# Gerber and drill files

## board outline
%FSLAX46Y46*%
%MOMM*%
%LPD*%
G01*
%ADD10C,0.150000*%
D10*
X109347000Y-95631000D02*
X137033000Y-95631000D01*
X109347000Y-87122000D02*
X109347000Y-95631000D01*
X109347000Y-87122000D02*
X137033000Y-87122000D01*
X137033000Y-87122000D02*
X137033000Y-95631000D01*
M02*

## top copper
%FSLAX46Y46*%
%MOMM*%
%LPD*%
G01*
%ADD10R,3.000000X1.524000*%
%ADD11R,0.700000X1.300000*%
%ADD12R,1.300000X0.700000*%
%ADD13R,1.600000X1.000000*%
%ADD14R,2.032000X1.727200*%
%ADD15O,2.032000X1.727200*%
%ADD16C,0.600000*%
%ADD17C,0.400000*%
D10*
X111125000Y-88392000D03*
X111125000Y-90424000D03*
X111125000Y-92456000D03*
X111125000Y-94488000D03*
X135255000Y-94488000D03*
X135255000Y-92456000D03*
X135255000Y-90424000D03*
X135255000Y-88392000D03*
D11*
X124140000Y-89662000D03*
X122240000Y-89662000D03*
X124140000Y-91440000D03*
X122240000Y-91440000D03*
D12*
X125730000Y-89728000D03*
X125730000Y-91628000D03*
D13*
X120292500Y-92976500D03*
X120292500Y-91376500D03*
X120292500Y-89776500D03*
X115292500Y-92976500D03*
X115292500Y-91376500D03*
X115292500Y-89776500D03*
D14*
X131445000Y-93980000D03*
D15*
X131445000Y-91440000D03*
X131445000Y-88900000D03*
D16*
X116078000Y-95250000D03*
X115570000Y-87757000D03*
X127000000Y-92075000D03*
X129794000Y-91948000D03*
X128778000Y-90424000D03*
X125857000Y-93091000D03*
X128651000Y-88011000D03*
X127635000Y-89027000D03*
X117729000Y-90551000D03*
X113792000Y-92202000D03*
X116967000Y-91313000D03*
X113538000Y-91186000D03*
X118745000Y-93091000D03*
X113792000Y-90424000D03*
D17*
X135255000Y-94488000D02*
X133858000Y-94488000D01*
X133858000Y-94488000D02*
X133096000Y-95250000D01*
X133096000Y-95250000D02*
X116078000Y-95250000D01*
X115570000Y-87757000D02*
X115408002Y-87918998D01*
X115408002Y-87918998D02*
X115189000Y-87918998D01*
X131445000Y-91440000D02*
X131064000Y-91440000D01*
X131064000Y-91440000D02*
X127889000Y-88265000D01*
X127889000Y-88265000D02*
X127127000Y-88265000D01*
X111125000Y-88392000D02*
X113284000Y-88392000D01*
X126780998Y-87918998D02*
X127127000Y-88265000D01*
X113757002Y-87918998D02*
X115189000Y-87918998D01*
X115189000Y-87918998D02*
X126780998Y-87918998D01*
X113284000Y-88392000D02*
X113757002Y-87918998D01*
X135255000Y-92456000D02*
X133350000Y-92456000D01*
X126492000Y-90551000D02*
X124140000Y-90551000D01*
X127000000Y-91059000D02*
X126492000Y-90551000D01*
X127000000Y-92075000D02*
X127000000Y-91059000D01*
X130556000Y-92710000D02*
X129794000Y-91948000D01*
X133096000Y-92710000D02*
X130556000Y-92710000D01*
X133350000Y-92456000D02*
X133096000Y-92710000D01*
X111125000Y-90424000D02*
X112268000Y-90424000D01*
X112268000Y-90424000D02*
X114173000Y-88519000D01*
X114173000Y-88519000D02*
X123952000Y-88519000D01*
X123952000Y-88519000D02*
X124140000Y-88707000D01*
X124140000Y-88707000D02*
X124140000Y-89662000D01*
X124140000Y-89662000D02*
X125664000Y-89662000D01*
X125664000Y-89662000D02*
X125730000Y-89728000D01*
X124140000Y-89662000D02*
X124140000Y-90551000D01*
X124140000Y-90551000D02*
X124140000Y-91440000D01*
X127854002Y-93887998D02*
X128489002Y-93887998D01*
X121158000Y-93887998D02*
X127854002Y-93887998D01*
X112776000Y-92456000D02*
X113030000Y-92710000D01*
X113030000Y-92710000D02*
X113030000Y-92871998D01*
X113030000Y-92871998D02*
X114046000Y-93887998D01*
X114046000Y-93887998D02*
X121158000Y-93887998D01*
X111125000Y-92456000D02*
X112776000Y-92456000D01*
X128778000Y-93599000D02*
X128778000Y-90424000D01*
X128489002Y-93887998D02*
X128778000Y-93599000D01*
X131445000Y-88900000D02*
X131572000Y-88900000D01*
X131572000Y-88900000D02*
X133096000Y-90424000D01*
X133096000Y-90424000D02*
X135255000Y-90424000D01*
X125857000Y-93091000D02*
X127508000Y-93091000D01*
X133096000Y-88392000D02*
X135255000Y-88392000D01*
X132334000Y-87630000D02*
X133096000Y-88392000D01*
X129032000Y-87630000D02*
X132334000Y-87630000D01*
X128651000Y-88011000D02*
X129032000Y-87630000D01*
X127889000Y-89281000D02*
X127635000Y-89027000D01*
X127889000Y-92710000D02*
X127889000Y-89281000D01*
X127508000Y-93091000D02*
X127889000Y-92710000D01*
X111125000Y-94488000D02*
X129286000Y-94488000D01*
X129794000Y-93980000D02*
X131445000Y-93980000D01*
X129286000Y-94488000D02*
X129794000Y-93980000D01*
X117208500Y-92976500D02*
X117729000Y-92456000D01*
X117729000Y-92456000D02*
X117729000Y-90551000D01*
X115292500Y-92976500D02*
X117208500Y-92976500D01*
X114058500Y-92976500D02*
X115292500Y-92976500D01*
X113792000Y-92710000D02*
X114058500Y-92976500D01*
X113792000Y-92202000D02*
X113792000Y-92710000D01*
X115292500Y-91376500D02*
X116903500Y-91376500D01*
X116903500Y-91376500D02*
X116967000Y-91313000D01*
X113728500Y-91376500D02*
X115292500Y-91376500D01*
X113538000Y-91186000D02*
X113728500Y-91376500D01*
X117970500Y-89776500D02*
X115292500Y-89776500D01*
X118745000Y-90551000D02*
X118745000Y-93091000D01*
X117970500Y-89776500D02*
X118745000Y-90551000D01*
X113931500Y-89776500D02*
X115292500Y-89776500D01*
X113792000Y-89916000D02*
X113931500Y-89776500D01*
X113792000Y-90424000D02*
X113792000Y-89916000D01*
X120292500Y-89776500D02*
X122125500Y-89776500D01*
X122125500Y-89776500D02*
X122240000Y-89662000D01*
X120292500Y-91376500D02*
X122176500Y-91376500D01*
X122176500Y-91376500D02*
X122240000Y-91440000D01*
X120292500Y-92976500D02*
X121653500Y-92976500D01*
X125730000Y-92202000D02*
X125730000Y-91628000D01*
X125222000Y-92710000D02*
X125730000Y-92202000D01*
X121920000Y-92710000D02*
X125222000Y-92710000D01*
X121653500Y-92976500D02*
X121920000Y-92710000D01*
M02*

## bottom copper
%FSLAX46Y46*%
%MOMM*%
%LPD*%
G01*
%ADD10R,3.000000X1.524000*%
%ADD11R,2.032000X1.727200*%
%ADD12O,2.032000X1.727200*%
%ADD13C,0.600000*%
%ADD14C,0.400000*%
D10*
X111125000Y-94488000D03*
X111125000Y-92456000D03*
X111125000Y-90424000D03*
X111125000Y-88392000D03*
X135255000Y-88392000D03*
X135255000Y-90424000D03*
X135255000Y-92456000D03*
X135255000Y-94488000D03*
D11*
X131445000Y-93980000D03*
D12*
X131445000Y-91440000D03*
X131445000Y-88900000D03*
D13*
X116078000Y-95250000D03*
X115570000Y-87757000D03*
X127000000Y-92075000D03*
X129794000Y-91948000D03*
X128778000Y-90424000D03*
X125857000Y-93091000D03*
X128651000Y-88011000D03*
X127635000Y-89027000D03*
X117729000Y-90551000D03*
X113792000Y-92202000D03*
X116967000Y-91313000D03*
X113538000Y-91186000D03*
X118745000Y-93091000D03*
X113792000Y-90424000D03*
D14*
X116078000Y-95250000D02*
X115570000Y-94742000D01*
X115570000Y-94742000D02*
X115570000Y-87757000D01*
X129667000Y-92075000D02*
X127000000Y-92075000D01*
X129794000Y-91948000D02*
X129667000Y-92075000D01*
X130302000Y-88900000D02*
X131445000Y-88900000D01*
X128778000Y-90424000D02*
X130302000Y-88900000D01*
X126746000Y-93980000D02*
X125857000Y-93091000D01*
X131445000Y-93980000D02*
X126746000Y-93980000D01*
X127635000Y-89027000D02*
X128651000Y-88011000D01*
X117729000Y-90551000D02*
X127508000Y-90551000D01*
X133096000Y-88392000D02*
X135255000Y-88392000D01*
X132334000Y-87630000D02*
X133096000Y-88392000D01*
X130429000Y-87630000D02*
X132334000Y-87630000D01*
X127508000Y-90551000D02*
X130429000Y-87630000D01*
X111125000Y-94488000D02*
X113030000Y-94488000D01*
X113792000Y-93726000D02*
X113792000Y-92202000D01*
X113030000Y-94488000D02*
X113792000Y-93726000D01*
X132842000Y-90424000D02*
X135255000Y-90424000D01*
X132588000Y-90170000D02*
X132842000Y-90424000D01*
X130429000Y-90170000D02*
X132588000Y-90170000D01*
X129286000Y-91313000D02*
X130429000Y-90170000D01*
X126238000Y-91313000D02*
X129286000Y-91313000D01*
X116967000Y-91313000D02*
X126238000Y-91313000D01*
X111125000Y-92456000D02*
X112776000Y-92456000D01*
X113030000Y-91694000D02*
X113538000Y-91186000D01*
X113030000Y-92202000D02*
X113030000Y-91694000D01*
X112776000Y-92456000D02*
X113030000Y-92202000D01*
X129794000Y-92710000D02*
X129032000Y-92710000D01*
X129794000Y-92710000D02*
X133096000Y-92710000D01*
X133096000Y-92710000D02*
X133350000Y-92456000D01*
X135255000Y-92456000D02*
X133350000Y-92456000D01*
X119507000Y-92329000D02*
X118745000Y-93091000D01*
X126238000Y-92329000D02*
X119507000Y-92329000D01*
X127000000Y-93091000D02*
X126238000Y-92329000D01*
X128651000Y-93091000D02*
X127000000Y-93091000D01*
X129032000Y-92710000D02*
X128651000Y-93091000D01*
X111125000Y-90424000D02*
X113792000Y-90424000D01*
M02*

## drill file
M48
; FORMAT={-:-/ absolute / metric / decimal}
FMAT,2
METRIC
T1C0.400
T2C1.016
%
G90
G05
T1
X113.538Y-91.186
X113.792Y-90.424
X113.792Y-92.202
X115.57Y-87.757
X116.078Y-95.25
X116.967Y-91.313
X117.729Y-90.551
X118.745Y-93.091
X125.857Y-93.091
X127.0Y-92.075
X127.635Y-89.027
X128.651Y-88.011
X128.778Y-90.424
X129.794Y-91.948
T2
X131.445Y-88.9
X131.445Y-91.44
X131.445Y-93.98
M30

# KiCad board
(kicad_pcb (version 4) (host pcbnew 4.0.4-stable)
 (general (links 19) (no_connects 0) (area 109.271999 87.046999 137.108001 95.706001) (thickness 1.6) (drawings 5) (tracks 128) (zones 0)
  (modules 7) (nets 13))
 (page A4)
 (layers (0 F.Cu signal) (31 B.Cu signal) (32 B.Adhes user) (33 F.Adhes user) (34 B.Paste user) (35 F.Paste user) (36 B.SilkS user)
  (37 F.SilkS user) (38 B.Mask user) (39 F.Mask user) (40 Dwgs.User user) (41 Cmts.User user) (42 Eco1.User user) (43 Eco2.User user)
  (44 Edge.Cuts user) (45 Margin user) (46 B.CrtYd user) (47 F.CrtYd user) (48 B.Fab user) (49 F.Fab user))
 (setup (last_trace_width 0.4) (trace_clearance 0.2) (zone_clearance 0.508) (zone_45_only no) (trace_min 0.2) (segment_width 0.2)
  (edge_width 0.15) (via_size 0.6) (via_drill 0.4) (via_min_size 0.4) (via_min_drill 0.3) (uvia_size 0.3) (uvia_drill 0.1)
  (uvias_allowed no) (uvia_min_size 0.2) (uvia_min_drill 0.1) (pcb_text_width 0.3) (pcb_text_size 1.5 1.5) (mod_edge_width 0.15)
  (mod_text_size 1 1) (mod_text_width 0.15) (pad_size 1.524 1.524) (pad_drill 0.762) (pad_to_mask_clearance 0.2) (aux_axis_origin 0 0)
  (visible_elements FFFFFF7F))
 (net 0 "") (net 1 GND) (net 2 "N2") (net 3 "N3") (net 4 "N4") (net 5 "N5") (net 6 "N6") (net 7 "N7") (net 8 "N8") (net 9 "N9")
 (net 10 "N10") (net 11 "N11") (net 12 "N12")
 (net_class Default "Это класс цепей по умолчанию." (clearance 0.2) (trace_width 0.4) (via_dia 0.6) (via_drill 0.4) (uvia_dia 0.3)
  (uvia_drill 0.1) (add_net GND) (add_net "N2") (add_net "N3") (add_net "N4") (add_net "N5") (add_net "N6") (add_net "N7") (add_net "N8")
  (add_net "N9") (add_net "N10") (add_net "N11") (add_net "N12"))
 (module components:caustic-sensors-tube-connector (layer F.Cu) (at 111.125 91.44 270)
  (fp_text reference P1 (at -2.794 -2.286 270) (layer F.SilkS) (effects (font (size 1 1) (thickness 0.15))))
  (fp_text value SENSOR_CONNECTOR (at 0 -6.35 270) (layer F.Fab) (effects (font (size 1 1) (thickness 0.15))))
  (pad 1 smd rect (at -3.048 0 270) (size 1.524 3) (layers F.Cu F.Paste F.Mask) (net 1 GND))
  (pad 2 smd rect (at -1.016 0 270) (size 1.524 3) (layers F.Cu F.Paste F.Mask) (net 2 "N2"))
  (pad 3 smd rect (at 1.016 0 270) (size 1.524 3) (layers F.Cu F.Paste F.Mask) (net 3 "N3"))
  (pad 4 smd rect (at 3.048 0 270) (size 1.524 3) (layers F.Cu F.Paste F.Mask) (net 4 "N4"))
  (pad 5 smd rect (at 3.048 0 270) (size 1.524 3) (layers B.Cu B.Paste B.Mask) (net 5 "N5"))
  (pad 6 smd rect (at 1.016 0 270) (size 1.524 3) (layers B.Cu B.Paste B.Mask) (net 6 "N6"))
  (pad 7 smd rect (at -1.016 0 270) (size 1.524 3) (layers B.Cu B.Paste B.Mask) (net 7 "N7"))
  (pad 8 smd rect (at -3.048 0 270) (size 1.524 3) (layers B.Cu B.Paste B.Mask) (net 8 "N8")))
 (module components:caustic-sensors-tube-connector (layer F.Cu) (at 135.255 91.44 90)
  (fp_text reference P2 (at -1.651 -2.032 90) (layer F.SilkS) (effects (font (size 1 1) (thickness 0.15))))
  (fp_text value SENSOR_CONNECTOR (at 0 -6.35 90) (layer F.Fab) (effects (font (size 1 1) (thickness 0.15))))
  (pad 1 smd rect (at -3.048 0 90) (size 1.524 3) (layers F.Cu F.Paste F.Mask) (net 1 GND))
  (pad 2 smd rect (at -1.016 0 90) (size 1.524 3) (layers F.Cu F.Paste F.Mask) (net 2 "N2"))
  (pad 3 smd rect (at 1.016 0 90) (size 1.524 3) (layers F.Cu F.Paste F.Mask) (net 3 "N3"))
  (pad 4 smd rect (at 3.048 0 90) (size 1.524 3) (layers F.Cu F.Paste F.Mask) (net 4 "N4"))
  (pad 5 smd rect (at 3.048 0 90) (size 1.524 3) (layers B.Cu B.Paste B.Mask) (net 5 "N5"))
  (pad 6 smd rect (at 1.016 0 90) (size 1.524 3) (layers B.Cu B.Paste B.Mask) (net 6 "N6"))
  (pad 7 smd rect (at -1.016 0 90) (size 1.524 3) (layers B.Cu B.Paste B.Mask) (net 7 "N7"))
  (pad 8 smd rect (at -3.048 0 90) (size 1.524 3) (layers B.Cu B.Paste B.Mask) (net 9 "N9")))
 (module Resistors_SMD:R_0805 (layer F.Cu) (at 123.19 89.662 180)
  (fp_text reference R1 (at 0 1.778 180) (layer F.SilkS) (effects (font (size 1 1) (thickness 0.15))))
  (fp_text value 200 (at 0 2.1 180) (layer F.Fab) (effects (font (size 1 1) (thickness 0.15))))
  (pad 1 smd rect (at -0.95 0 180) (size 0.7 1.3) (layers F.Cu F.Paste F.Mask) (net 2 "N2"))
  (pad 2 smd rect (at 0.95 0 180) (size 0.7 1.3) (layers F.Cu F.Paste F.Mask) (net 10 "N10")))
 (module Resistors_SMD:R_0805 (layer F.Cu) (at 123.19 91.44 180)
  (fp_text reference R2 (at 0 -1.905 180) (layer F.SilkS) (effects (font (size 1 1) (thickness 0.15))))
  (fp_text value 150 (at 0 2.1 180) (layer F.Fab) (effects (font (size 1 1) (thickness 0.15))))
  (pad 1 smd rect (at -0.95 0 180) (size 0.7 1.3) (layers F.Cu F.Paste F.Mask) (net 2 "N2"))
  (pad 2 smd rect (at 0.95 0 180) (size 0.7 1.3) (layers F.Cu F.Paste F.Mask) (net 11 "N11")))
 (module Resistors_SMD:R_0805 (layer F.Cu) (at 125.73 90.678 270)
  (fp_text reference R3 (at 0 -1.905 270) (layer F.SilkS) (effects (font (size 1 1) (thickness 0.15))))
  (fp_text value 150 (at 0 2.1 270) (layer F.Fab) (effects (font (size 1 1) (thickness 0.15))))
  (pad 1 smd rect (at -0.95 0 270) (size 0.7 1.3) (layers F.Cu F.Paste F.Mask) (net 2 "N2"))
  (pad 2 smd rect (at 0.95 0 270) (size 0.7 1.3) (layers F.Cu F.Paste F.Mask) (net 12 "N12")))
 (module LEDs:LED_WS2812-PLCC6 (layer F.Cu) (at 117.7925 91.3765)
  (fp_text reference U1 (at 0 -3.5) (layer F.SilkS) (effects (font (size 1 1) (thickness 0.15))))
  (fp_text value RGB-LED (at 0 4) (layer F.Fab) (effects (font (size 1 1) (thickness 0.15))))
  (pad 4 smd rect (at 2.5 1.6) (size 1.6 1) (layers F.Cu F.Paste F.Mask) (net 12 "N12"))
  (pad 5 smd rect (at 2.5 0) (size 1.6 1) (layers F.Cu F.Paste F.Mask) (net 11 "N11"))
  (pad 6 smd rect (at 2.5 -1.6) (size 1.6 1) (layers F.Cu F.Paste F.Mask) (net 10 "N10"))
  (pad 3 smd rect (at -2.5 1.6) (size 1.6 1) (layers F.Cu F.Paste F.Mask) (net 5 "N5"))
  (pad 2 smd rect (at -2.5 0) (size 1.6 1) (layers F.Cu F.Paste F.Mask) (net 6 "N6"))
  (pad 1 smd rect (at -2.5 -1.6) (size 1.6 1) (layers F.Cu F.Paste F.Mask) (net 7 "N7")))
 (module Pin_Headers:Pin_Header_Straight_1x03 (layer F.Cu) (at 131.445 93.98 180)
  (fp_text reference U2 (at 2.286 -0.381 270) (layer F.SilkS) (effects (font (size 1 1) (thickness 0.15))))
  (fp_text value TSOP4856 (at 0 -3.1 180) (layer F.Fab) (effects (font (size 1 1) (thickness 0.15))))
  (pad 1 thru_hole rect (at 0 0 180) (size 2.032 1.7272) (drill 1.016) (layers *.Cu *.Mask) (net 4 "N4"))
  (pad 2 thru_hole oval (at 0 2.54 180) (size 2.032 1.7272) (drill 1.016) (layers *.Cu *.Mask) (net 1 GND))
  (pad 3 thru_hole oval (at 0 5.08 180) (size 2.032 1.7272) (drill 1.016) (layers *.Cu *.Mask) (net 3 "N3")))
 (gr_line (start 109.347 95.631) (end 137.033 95.631) (angle 90) (layer Edge.Cuts) (width 0.15))
 (gr_line (start 109.347 87.122) (end 109.347 95.631) (angle 90) (layer Edge.Cuts) (width 0.15))
 (gr_line (start 109.347 87.122) (end 137.033 87.122) (angle 90) (layer Edge.Cuts) (width 0.15))
 (gr_line (start 137.033 87.122) (end 137.033 95.631) (angle 90) (layer Edge.Cuts) (width 0.15))
 (segment (start 135.255 94.488) (end 133.858 94.488) (width 0.4) (layer F.Cu) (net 1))
 (segment (start 133.858 94.488) (end 133.096 95.25) (width 0.4) (layer F.Cu) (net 1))
 (segment (start 133.096 95.25) (end 116.078 95.25) (width 0.4) (layer F.Cu) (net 1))
 (via (at 116.078 95.25) (size 0.6) (drill 0.4) (layers F.Cu B.Cu) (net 1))
 (segment (start 116.078 95.25) (end 115.57 94.742) (width 0.4) (layer B.Cu) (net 1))
 (segment (start 115.57 94.742) (end 115.57 87.757) (width 0.4) (layer B.Cu) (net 1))
 (via (at 115.57 87.757) (size 0.6) (drill 0.4) (layers F.Cu B.Cu) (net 1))
 (segment (start 115.57 87.757) (end 115.408002 87.918998) (width 0.4) (layer F.Cu) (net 1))
 (segment (start 115.408002 87.918998) (end 115.189 87.918998) (width 0.4) (layer F.Cu) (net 1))
 (segment (start 131.445 91.44) (end 131.064 91.44) (width 0.4) (layer F.Cu) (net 1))
 (segment (start 131.064 91.44) (end 127.889 88.265) (width 0.4) (layer F.Cu) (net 1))
 (segment (start 127.889 88.265) (end 127.127 88.265) (width 0.4) (layer F.Cu) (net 1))
 (segment (start 111.125 88.392) (end 113.284 88.392) (width 0.4) (layer F.Cu) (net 1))
 (segment (start 126.780998 87.918998) (end 127.127 88.265) (width 0.4) (layer F.Cu) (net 1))
 (segment (start 113.757002 87.918998) (end 115.189 87.918998) (width 0.4) (layer F.Cu) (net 1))
 (segment (start 115.189 87.918998) (end 126.780998 87.918998) (width 0.4) (layer F.Cu) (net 1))
 (segment (start 113.284 88.392) (end 113.757002 87.918998) (width 0.4) (layer F.Cu) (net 1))
 (segment (start 135.255 92.456) (end 133.35 92.456) (width 0.4) (layer F.Cu) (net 2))
 (segment (start 126.492 90.551) (end 124.14 90.551) (width 0.4) (layer F.Cu) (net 2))
 (segment (start 127 91.059) (end 126.492 90.551) (width 0.4) (layer F.Cu) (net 2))
 (segment (start 127 92.075) (end 127 91.059) (width 0.4) (layer F.Cu) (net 2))
 (via (at 127 92.075) (size 0.6) (drill 0.4) (layers F.Cu B.Cu) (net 2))
 (segment (start 129.667 92.075) (end 127 92.075) (width 0.4) (layer B.Cu) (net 2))
 (segment (start 129.794 91.948) (end 129.667 92.075) (width 0.4) (layer B.Cu) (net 2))
 (via (at 129.794 91.948) (size 0.6) (drill 0.4) (layers F.Cu B.Cu) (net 2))
 (segment (start 130.556 92.71) (end 129.794 91.948) (width 0.4) (layer F.Cu) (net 2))
 (segment (start 133.096 92.71) (end 130.556 92.71) (width 0.4) (layer F.Cu) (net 2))
 (segment (start 133.35 92.456) (end 133.096 92.71) (width 0.4) (layer F.Cu) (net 2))
 (segment (start 111.125 90.424) (end 112.268 90.424) (width 0.4) (layer F.Cu) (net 2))
 (segment (start 112.268 90.424) (end 114.173 88.519) (width 0.4) (layer F.Cu) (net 2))
 (segment (start 114.173 88.519) (end 123.952 88.519) (width 0.4) (layer F.Cu) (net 2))
 (segment (start 123.952 88.519) (end 124.14 88.707) (width 0.4) (layer F.Cu) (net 2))
 (segment (start 124.14 88.707) (end 124.14 89.662) (width 0.4) (layer F.Cu) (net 2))
 (segment (start 124.14 89.662) (end 125.664 89.662) (width 0.4) (layer F.Cu) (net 2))
 (segment (start 125.664 89.662) (end 125.73 89.728) (width 0.4) (layer F.Cu) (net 2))
 (segment (start 124.14 89.662) (end 124.14 90.551) (width 0.4) (layer F.Cu) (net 2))
 (segment (start 124.14 90.551) (end 124.14 91.44) (width 0.4) (layer F.Cu) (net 2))
 (segment (start 127.854002 93.887998) (end 128.489002 93.887998) (width 0.4) (layer F.Cu) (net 3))
 (segment (start 121.158 93.887998) (end 127.854002 93.887998) (width 0.4) (layer F.Cu) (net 3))
 (segment (start 112.776 92.456) (end 113.03 92.71) (width 0.4) (layer F.Cu) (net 3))
 (segment (start 113.03 92.71) (end 113.03 92.871998) (width 0.4) (layer F.Cu) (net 3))
 (segment (start 113.03 92.871998) (end 114.046 93.887998) (width 0.4) (layer F.Cu) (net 3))
 (segment (start 114.046 93.887998) (end 121.158 93.887998) (width 0.4) (layer F.Cu) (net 3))
 (segment (start 111.125 92.456) (end 112.776 92.456) (width 0.4) (layer F.Cu) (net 3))
 (segment (start 130.302 88.9) (end 131.445 88.9) (width 0.4) (layer B.Cu) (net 3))
 (segment (start 128.778 90.424) (end 130.302 88.9) (width 0.4) (layer B.Cu) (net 3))
 (via (at 128.778 90.424) (size 0.6) (drill 0.4) (layers F.Cu B.Cu) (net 3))
 (segment (start 128.778 93.599) (end 128.778 90.424) (width 0.4) (layer F.Cu) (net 3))
 (segment (start 128.489002 93.887998) (end 128.778 93.599) (width 0.4) (layer F.Cu) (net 3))
 (segment (start 131.445 88.9) (end 131.572 88.9) (width 0.4) (layer F.Cu) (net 3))
 (segment (start 131.572 88.9) (end 133.096 90.424) (width 0.4) (layer F.Cu) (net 3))
 (segment (start 133.096 90.424) (end 135.255 90.424) (width 0.4) (layer F.Cu) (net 3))
 (segment (start 125.857 93.091) (end 127.508 93.091) (width 0.4) (layer F.Cu) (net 4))
 (segment (start 126.746 93.98) (end 125.857 93.091) (width 0.4) (layer B.Cu) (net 4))
 (via (at 125.857 93.091) (size 0.6) (drill 0.4) (layers F.Cu B.Cu) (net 4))
 (segment (start 131.445 93.98) (end 126.746 93.98) (width 0.4) (layer B.Cu) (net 4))
 (segment (start 133.096 88.392) (end 135.255 88.392) (width 0.4) (layer F.Cu) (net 4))
 (segment (start 132.334 87.63) (end 133.096 88.392) (width 0.4) (layer F.Cu) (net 4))
 (segment (start 129.032 87.63) (end 132.334 87.63) (width 0.4) (layer F.Cu) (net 4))
 (segment (start 128.651 88.011) (end 129.032 87.63) (width 0.4) (layer F.Cu) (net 4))
 (via (at 128.651 88.011) (size 0.6) (drill 0.4) (layers F.Cu B.Cu) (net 4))
 (segment (start 127.635 89.027) (end 128.651 88.011) (width 0.4) (layer B.Cu) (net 4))
 (via (at 127.635 89.027) (size 0.6) (drill 0.4) (layers F.Cu B.Cu) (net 4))
 (segment (start 127.889 89.281) (end 127.635 89.027) (width 0.4) (layer F.Cu) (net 4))
 (segment (start 127.889 92.71) (end 127.889 89.281) (width 0.4) (layer F.Cu) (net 4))
 (segment (start 127.508 93.091) (end 127.889 92.71) (width 0.4) (layer F.Cu) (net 4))
 (segment (start 111.125 94.488) (end 129.286 94.488) (width 0.4) (layer F.Cu) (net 4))
 (segment (start 129.794 93.98) (end 131.445 93.98) (width 0.4) (layer F.Cu) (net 4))
 (segment (start 129.286 94.488) (end 129.794 93.98) (width 0.4) (layer F.Cu) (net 4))
 (segment (start 117.729 90.551) (end 127.508 90.551) (width 0.4) (layer B.Cu) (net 5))
 (segment (start 117.2085 92.9765) (end 117.729 92.456) (width 0.4) (layer F.Cu) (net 5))
 (segment (start 117.729 92.456) (end 117.729 90.551) (width 0.4) (layer F.Cu) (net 5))
 (via (at 117.729 90.551) (size 0.6) (drill 0.4) (layers F.Cu B.Cu) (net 5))
 (segment (start 115.2925 92.9765) (end 117.2085 92.9765) (width 0.4) (layer F.Cu) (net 5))
 (segment (start 133.096 88.392) (end 135.255 88.392) (width 0.4) (layer B.Cu) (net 5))
 (segment (start 132.334 87.63) (end 133.096 88.392) (width 0.4) (layer B.Cu) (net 5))
 (segment (start 130.429 87.63) (end 132.334 87.63) (width 0.4) (layer B.Cu) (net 5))
 (segment (start 127.508 90.551) (end 130.429 87.63) (width 0.4) (layer B.Cu) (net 5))
 (segment (start 111.125 94.488) (end 113.03 94.488) (width 0.4) (layer B.Cu) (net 5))
 (segment (start 114.0585 92.9765) (end 115.2925 92.9765) (width 0.4) (layer F.Cu) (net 5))
 (segment (start 113.792 92.71) (end 114.0585 92.9765) (width 0.4) (layer F.Cu) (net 5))
 (segment (start 113.792 92.202) (end 113.792 92.71) (width 0.4) (layer F.Cu) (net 5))
 (via (at 113.792 92.202) (size 0.6) (drill 0.4) (layers F.Cu B.Cu) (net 5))
 (segment (start 113.792 93.726) (end 113.792 92.202) (width 0.4) (layer B.Cu) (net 5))
 (segment (start 113.03 94.488) (end 113.792 93.726) (width 0.4) (layer B.Cu) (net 5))
 (segment (start 115.2925 91.3765) (end 116.9035 91.3765) (width 0.4) (layer F.Cu) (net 6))
 (segment (start 132.842 90.424) (end 135.255 90.424) (width 0.4) (layer B.Cu) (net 6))
 (segment (start 132.588 90.17) (end 132.842 90.424) (width 0.4) (layer B.Cu) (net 6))
 (segment (start 130.429 90.17) (end 132.588 90.17) (width 0.4) (layer B.Cu) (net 6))
 (segment (start 129.286 91.313) (end 130.429 90.17) (width 0.4) (layer B.Cu) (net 6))
 (segment (start 126.238 91.313) (end 129.286 91.313) (width 0.4) (layer B.Cu) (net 6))
 (segment (start 116.967 91.313) (end 126.238 91.313) (width 0.4) (layer B.Cu) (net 6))
 (via (at 116.967 91.313) (size 0.6) (drill 0.4) (layers F.Cu B.Cu) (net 6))
 (segment (start 116.9035 91.3765) (end 116.967 91.313) (width 0.4) (layer F.Cu) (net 6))
 (segment (start 111.125 92.456) (end 112.776 92.456) (width 0.4) (layer B.Cu) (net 6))
 (segment (start 113.7285 91.3765) (end 115.2925 91.3765) (width 0.4) (layer F.Cu) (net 6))
 (segment (start 113.538 91.186) (end 113.7285 91.3765) (width 0.4) (layer F.Cu) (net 6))
 (via (at 113.538 91.186) (size 0.6) (drill 0.4) (layers F.Cu B.Cu) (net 6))
 (segment (start 113.03 91.694) (end 113.538 91.186) (width 0.4) (layer B.Cu) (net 6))
 (segment (start 113.03 92.202) (end 113.03 91.694) (width 0.4) (layer B.Cu) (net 6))
 (segment (start 112.776 92.456) (end 113.03 92.202) (width 0.4) (layer B.Cu) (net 6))
 (segment (start 129.794 92.71) (end 129.032 92.71) (width 0.4) (layer B.Cu) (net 7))
 (segment (start 129.794 92.71) (end 133.096 92.71) (width 0.4) (layer B.Cu) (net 7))
 (segment (start 133.096 92.71) (end 133.35 92.456) (width 0.4) (layer B.Cu) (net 7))
 (segment (start 135.255 92.456) (end 133.35 92.456) (width 0.4) (layer B.Cu) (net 7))
 (segment (start 117.9705 89.7765) (end 115.2925 89.7765) (width 0.4) (layer F.Cu) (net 7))
 (via (at 118.745 93.091) (size 0.6) (drill 0.4) (layers F.Cu B.Cu) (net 7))
 (segment (start 118.745 90.551) (end 118.745 93.091) (width 0.4) (layer F.Cu) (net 7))
 (segment (start 117.9705 89.7765) (end 118.745 90.551) (width 0.4) (layer F.Cu) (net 7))
 (segment (start 119.507 92.329) (end 118.745 93.091) (width 0.4) (layer B.Cu) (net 7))
 (segment (start 126.238 92.329) (end 119.507 92.329) (width 0.4) (layer B.Cu) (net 7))
 (segment (start 127 93.091) (end 126.238 92.329) (width 0.4) (layer B.Cu) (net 7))
 (segment (start 128.651 93.091) (end 127 93.091) (width 0.4) (layer B.Cu) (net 7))
 (segment (start 129.032 92.71) (end 128.651 93.091) (width 0.4) (layer B.Cu) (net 7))
 (segment (start 111.125 90.424) (end 113.792 90.424) (width 0.4) (layer B.Cu) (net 7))
 (segment (start 113.9315 89.7765) (end 115.2925 89.7765) (width 0.4) (layer F.Cu) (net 7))
 (segment (start 113.792 89.916) (end 113.9315 89.7765) (width 0.4) (layer F.Cu) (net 7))
 (segment (start 113.792 90.424) (end 113.792 89.916) (width 0.4) (layer F.Cu) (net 7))
 (via (at 113.792 90.424) (size 0.6) (drill 0.4) (layers F.Cu B.Cu) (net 7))
 (segment (start 120.2925 89.7765) (end 122.1255 89.7765) (width 0.4) (layer F.Cu) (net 10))
 (segment (start 122.1255 89.7765) (end 122.24 89.662) (width 0.4) (layer F.Cu) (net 10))
 (segment (start 120.2925 91.3765) (end 122.1765 91.3765) (width 0.4) (layer F.Cu) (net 11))
 (segment (start 122.1765 91.3765) (end 122.24 91.44) (width 0.4) (layer F.Cu) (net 11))
 (segment (start 120.2925 92.9765) (end 121.6535 92.9765) (width 0.4) (layer F.Cu) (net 12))
 (segment (start 125.73 92.202) (end 125.73 91.628) (width 0.4) (layer F.Cu) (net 12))
 (segment (start 125.222 92.71) (end 125.73 92.202) (width 0.4) (layer F.Cu) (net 12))
 (segment (start 121.92 92.71) (end 125.222 92.71) (width 0.4) (layer F.Cu) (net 12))
 (segment (start 121.6535 92.9765) (end 121.92 92.71) (width 0.4) (layer F.Cu) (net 12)))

